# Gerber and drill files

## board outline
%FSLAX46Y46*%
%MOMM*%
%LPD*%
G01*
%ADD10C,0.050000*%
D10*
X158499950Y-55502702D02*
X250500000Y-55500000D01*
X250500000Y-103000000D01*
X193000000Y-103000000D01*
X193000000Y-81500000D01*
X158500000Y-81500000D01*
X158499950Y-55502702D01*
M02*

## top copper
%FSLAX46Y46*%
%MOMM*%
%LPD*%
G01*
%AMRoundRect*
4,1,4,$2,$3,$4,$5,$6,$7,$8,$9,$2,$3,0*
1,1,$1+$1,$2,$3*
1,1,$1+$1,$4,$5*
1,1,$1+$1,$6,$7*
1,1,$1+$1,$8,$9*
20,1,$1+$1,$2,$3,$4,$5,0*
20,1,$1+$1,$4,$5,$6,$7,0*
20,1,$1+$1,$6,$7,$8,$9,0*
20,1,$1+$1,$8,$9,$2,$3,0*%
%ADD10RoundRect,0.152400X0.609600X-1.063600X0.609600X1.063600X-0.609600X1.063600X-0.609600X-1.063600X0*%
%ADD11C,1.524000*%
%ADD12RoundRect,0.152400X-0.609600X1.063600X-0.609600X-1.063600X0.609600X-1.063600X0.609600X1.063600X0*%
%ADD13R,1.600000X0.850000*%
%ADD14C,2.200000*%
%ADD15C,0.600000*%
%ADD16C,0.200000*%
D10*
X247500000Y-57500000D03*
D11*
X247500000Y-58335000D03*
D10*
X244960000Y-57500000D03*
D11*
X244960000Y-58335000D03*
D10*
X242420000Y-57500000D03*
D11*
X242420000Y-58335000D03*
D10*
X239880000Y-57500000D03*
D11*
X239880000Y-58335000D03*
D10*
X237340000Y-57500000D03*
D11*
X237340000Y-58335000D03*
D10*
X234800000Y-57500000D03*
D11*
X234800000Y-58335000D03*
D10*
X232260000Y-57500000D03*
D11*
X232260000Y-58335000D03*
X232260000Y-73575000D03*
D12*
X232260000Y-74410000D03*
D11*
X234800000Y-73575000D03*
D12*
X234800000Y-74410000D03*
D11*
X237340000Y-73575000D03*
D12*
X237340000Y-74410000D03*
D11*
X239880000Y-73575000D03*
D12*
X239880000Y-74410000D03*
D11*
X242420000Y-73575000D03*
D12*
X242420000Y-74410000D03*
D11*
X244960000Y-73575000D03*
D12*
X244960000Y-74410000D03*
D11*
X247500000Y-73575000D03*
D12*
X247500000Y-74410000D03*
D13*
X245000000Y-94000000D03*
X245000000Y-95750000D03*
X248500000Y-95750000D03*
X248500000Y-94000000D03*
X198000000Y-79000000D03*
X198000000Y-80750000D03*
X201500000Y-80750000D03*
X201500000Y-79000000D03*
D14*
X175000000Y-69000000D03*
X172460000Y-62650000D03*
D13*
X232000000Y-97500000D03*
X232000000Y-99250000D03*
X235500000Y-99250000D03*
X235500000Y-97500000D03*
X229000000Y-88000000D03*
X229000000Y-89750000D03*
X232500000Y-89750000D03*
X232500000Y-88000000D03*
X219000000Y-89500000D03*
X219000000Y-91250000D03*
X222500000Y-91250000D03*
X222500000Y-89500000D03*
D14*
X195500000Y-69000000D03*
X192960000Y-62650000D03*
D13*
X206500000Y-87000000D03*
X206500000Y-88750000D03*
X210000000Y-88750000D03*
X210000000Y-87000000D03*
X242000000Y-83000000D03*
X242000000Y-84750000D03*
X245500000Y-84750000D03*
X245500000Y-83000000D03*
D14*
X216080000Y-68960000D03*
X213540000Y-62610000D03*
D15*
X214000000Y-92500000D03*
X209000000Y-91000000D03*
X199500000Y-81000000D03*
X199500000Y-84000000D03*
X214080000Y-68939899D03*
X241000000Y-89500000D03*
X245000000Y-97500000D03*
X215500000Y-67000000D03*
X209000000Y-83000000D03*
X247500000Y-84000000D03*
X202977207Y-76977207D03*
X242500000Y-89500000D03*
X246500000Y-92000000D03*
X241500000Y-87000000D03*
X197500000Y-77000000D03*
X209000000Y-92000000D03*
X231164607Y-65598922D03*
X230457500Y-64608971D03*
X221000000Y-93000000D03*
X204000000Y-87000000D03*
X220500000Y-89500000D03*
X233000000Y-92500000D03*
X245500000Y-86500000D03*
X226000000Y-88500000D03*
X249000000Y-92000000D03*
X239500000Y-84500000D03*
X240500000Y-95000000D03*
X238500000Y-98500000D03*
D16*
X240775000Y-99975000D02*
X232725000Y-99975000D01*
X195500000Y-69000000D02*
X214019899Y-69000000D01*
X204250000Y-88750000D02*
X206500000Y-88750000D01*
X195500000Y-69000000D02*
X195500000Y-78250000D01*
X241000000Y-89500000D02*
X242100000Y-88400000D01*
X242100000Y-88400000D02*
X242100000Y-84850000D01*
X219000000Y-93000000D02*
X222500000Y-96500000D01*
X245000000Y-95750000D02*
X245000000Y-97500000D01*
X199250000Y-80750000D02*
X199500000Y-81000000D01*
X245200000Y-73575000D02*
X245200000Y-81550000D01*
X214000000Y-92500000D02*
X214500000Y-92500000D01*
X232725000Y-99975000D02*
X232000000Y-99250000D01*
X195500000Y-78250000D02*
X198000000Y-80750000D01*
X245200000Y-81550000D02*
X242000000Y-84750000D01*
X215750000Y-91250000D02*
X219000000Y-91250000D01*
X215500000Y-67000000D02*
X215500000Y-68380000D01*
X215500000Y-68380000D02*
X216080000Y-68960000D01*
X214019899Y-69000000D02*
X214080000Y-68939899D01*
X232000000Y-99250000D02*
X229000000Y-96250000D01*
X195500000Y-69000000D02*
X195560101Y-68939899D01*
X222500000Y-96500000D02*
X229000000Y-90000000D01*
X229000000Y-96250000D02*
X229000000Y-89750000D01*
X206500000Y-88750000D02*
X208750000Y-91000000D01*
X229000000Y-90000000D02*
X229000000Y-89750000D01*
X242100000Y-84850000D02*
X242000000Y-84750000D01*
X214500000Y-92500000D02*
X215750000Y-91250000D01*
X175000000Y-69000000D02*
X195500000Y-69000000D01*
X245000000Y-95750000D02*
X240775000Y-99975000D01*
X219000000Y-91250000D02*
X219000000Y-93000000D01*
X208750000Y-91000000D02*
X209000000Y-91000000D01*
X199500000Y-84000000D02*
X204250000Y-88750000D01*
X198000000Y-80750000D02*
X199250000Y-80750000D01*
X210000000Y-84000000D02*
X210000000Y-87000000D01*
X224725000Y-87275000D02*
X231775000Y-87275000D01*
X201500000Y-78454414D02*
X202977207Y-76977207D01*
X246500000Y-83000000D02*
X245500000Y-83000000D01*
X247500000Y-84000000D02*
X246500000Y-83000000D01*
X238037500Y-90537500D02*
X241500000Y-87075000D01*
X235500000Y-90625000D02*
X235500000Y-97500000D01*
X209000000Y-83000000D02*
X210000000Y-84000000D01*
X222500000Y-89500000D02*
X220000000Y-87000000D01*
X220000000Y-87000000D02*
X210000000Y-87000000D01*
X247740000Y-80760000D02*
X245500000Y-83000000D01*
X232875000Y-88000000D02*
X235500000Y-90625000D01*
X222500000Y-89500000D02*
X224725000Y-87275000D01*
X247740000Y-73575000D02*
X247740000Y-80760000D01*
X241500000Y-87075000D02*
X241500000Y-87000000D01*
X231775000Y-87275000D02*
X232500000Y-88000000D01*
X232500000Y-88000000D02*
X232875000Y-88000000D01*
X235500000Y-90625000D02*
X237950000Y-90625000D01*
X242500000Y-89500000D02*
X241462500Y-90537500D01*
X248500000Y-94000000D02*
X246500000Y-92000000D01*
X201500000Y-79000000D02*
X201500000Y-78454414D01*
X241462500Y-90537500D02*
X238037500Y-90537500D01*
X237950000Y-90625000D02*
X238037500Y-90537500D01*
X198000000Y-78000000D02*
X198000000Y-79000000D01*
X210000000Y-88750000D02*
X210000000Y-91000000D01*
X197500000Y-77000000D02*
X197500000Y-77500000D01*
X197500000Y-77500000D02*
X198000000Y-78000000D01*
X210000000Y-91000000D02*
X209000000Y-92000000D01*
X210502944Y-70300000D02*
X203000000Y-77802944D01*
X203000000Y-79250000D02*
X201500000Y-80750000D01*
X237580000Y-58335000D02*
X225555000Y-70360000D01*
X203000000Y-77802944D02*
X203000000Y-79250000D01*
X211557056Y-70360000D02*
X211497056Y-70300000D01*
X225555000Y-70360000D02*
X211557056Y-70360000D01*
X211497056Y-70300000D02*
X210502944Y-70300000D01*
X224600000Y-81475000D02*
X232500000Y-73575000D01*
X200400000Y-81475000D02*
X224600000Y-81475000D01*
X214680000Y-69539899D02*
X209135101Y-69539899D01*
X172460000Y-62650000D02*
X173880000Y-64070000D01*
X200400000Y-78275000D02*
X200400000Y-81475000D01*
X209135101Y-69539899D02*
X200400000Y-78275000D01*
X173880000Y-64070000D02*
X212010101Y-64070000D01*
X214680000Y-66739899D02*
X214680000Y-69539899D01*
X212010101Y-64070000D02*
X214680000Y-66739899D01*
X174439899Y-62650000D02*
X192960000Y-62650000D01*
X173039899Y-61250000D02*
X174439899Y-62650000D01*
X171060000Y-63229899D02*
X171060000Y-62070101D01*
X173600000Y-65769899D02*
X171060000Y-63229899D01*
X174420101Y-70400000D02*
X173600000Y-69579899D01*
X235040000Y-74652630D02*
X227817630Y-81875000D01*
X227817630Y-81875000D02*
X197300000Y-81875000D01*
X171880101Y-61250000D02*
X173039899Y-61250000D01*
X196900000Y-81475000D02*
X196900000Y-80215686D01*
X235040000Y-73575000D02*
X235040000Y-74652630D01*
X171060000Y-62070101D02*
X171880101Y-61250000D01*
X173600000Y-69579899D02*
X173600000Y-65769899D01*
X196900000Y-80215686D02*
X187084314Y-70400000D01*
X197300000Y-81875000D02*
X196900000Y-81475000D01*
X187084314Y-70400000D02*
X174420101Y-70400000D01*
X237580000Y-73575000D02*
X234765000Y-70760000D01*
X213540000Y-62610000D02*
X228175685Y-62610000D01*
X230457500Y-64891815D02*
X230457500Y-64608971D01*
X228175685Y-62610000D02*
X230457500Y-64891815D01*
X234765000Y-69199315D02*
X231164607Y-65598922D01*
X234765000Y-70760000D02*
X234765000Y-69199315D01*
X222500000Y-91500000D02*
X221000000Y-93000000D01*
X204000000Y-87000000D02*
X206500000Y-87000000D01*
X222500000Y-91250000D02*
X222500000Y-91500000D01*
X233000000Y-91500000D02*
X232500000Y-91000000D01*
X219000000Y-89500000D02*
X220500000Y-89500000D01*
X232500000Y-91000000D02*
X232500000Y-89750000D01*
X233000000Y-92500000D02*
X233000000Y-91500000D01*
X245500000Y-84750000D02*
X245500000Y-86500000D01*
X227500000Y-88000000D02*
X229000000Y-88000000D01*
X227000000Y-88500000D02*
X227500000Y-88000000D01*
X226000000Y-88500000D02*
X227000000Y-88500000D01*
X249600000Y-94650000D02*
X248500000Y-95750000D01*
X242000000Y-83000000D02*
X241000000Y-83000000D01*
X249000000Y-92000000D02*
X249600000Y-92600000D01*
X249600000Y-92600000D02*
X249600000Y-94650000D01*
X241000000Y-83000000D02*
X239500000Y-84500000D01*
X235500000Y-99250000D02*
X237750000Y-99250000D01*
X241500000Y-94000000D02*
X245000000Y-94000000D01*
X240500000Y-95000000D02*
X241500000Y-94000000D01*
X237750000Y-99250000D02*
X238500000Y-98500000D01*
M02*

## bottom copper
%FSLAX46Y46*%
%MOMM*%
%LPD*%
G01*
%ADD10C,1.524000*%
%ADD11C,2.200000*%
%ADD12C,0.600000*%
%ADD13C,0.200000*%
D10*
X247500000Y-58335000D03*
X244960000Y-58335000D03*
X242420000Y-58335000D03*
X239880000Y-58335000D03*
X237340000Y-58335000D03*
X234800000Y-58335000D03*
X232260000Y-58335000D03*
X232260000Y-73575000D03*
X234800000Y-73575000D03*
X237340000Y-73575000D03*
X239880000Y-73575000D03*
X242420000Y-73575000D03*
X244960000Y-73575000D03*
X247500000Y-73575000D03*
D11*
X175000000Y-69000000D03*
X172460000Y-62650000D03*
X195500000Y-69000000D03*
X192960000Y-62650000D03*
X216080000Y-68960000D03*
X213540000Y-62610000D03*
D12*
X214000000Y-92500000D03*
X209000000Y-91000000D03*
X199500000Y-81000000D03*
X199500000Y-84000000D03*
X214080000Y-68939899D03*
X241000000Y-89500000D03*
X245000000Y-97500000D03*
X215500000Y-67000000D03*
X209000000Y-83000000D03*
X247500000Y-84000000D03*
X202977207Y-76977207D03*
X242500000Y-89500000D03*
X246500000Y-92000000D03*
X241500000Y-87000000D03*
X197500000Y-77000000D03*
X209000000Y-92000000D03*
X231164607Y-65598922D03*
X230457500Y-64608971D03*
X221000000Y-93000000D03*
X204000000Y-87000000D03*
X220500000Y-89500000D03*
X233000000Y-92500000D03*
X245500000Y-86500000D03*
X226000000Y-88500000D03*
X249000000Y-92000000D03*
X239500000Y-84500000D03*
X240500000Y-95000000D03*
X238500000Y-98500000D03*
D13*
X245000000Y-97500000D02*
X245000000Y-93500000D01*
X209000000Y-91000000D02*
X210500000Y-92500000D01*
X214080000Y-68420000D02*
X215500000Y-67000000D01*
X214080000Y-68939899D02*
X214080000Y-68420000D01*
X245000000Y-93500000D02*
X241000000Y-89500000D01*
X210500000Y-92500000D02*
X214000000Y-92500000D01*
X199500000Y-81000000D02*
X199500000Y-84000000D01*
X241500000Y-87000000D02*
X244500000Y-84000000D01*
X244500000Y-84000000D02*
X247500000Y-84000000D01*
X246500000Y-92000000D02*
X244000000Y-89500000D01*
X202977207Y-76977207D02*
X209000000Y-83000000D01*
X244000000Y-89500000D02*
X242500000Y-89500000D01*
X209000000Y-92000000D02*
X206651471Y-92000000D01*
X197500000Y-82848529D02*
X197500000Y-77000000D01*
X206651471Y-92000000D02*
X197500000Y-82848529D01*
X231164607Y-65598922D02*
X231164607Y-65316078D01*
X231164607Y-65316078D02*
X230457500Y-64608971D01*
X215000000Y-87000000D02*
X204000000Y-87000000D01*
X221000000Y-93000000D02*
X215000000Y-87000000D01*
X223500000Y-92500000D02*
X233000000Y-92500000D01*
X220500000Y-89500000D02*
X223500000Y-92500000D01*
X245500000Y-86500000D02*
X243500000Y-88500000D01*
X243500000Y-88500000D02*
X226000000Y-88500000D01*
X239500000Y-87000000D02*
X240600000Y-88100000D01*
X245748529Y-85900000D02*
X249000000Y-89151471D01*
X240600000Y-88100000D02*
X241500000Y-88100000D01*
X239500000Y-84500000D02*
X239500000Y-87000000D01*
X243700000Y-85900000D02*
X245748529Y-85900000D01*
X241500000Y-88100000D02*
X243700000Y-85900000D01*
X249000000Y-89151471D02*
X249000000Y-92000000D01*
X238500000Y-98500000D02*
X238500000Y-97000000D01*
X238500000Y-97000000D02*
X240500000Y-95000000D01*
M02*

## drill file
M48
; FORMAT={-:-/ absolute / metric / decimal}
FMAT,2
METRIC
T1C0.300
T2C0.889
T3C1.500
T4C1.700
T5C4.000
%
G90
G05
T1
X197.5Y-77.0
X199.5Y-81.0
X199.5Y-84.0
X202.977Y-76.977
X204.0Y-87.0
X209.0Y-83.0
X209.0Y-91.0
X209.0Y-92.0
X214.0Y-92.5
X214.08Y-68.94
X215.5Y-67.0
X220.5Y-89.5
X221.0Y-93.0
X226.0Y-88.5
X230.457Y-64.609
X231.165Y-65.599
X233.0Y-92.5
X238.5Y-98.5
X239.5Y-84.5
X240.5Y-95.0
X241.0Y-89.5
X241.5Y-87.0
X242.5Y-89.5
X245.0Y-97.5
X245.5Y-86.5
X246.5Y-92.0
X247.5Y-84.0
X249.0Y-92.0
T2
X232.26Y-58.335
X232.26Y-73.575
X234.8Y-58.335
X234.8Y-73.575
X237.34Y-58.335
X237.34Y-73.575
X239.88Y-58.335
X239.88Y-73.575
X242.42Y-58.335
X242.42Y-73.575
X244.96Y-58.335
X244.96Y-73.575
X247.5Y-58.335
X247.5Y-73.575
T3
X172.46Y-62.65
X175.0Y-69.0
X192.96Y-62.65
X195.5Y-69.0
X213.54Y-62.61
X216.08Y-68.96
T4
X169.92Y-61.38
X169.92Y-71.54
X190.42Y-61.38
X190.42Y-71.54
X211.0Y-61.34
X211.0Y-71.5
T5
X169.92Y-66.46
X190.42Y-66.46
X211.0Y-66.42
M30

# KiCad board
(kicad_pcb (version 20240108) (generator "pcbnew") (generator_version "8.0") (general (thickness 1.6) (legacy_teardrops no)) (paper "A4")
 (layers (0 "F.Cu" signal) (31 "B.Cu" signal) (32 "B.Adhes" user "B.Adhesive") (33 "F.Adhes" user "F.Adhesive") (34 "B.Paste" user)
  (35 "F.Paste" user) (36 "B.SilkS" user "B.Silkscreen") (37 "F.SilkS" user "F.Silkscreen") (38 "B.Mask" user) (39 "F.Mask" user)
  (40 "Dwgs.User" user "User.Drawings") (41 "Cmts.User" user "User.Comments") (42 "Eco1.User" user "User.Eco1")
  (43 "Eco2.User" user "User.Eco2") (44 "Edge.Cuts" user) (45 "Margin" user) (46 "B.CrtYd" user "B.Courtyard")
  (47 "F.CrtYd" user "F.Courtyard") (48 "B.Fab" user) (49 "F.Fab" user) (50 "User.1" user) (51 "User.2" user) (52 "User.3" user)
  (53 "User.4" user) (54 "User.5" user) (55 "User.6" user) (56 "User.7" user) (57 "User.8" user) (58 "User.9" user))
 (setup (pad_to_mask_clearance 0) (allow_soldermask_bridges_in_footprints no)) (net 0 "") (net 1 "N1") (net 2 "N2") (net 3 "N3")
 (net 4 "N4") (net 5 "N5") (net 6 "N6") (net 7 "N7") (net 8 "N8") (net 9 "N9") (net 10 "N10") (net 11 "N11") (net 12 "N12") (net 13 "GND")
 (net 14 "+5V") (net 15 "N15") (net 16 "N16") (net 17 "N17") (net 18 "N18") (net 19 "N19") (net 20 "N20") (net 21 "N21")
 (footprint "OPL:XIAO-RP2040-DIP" (layer "F.Cu") (at 239.88 65.955 -90)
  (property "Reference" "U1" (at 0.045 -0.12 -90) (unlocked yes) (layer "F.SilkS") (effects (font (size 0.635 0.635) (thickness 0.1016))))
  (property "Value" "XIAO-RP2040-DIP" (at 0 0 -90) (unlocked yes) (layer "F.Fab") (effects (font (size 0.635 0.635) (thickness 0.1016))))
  (pad "1" smd roundrect (at -8.455 -7.62 90) (size 2.432 1.524) (layers "F.Cu" "F.Mask") (roundrect_rratio 0.1) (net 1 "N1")
   (thermal_bridge_angle 45))
  (pad "1" thru_hole circle (at -7.62 -7.62 90) (size 1.524 1.524) (drill 0.889) (layers "*.Cu" "*.Mask") (remove_unused_layers no)
   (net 1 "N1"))
  (pad "2" smd roundrect (at -8.455 -5.08 90) (size 2.432 1.524) (layers "F.Cu" "F.Mask") (roundrect_rratio 0.1) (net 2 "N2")
   (thermal_bridge_angle 45))
  (pad "2" thru_hole circle (at -7.62 -5.08 90) (size 1.524 1.524) (drill 0.889) (layers "*.Cu" "*.Mask") (remove_unused_layers no)
   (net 2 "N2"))
  (pad "3" smd roundrect (at -8.455 -2.54 90) (size 2.432 1.524) (layers "F.Cu" "F.Mask") (roundrect_rratio 0.1) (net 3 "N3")
   (thermal_bridge_angle 45))
  (pad "3" thru_hole circle (at -7.62 -2.54 90) (size 1.524 1.524) (drill 0.889) (layers "*.Cu" "*.Mask") (remove_unused_layers no)
   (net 3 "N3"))
  (pad "4" smd roundrect (at -8.455 0 90) (size 2.432 1.524) (layers "F.Cu" "F.Mask") (roundrect_rratio 0.1) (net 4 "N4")
   (thermal_bridge_angle 45))
  (pad "4" thru_hole circle (at -7.62 0 90) (size 1.524 1.524) (drill 0.889) (layers "*.Cu" "*.Mask") (remove_unused_layers no) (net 4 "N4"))
  (pad "5" smd roundrect (at -8.455 2.54 90) (size 2.432 1.524) (layers "F.Cu" "F.Mask") (roundrect_rratio 0.1) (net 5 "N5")
   (thermal_bridge_angle 45))
  (pad "5" thru_hole circle (at -7.62 2.54 90) (size 1.524 1.524) (drill 0.889) (layers "*.Cu" "*.Mask") (remove_unused_layers no)
   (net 5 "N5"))
  (pad "6" smd roundrect (at -8.455 5.08 90) (size 2.432 1.524) (layers "F.Cu" "F.Mask") (roundrect_rratio 0.1) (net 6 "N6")
   (thermal_bridge_angle 45))
  (pad "6" thru_hole circle (at -7.62 5.08 90) (size 1.524 1.524) (drill 0.889) (layers "*.Cu" "*.Mask") (remove_unused_layers no)
   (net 6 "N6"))
  (pad "7" smd roundrect (at -8.455 7.62 90) (size 2.432 1.524) (layers "F.Cu" "F.Mask") (roundrect_rratio 0.1) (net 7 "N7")
   (thermal_bridge_angle 45))
  (pad "7" thru_hole circle (at -7.62 7.62 90) (size 1.524 1.524) (drill 0.889) (layers "*.Cu" "*.Mask") (remove_unused_layers no)
   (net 7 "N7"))
  (pad "8" thru_hole circle (at 7.62 7.62 270) (size 1.524 1.524) (drill 0.889) (layers "*.Cu" "*.Mask") (remove_unused_layers no)
   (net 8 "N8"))
  (pad "8" smd roundrect (at 8.455 7.62 270) (size 2.432 1.524) (layers "F.Cu" "F.Mask") (roundrect_rratio 0.1) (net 8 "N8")
   (thermal_bridge_angle 45))
  (pad "9" thru_hole circle (at 7.62 5.08 270) (size 1.524 1.524) (drill 0.889) (layers "*.Cu" "*.Mask") (remove_unused_layers no)
   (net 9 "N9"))
  (pad "9" smd roundrect (at 8.455 5.08 270) (size 2.432 1.524) (layers "F.Cu" "F.Mask") (roundrect_rratio 0.1) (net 9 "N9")
   (thermal_bridge_angle 45))
  (pad "10" thru_hole circle (at 7.62 2.54 270) (size 1.524 1.524) (drill 0.889) (layers "*.Cu" "*.Mask") (remove_unused_layers no)
   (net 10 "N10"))
  (pad "10" smd roundrect (at 8.455 2.54 270) (size 2.432 1.524) (layers "F.Cu" "F.Mask") (roundrect_rratio 0.1) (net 10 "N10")
   (thermal_bridge_angle 45))
  (pad "11" thru_hole circle (at 7.62 0 270) (size 1.524 1.524) (drill 0.889) (layers "*.Cu" "*.Mask") (remove_unused_layers no)
   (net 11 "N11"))
  (pad "11" smd roundrect (at 8.455 0 270) (size 2.432 1.524) (layers "F.Cu" "F.Mask") (roundrect_rratio 0.1) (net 11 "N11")
   (thermal_bridge_angle 45))
  (pad "12" thru_hole circle (at 7.62 -2.54 270) (size 1.524 1.524) (drill 0.889) (layers "*.Cu" "*.Mask") (remove_unused_layers no)
   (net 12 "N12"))
  (pad "12" smd roundrect (at 8.455 -2.54 270) (size 2.432 1.524) (layers "F.Cu" "F.Mask") (roundrect_rratio 0.1) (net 12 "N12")
   (thermal_bridge_angle 45))
  (pad "13" thru_hole circle (at 7.62 -5.08 270) (size 1.524 1.524) (drill 0.889) (layers "*.Cu" "*.Mask") (remove_unused_layers no)
   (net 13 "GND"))
  (pad "13" smd roundrect (at 8.455 -5.08 270) (size 2.432 1.524) (layers "F.Cu" "F.Mask") (roundrect_rratio 0.1) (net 13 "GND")
   (thermal_bridge_angle 45))
  (pad "14" thru_hole circle (at 7.62 -7.62 270) (size 1.524 1.524) (drill 0.889) (layers "*.Cu" "*.Mask") (remove_unused_layers no)
   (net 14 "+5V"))
  (pad "14" smd roundrect (at 8.455 -7.62 270) (size 2.432 1.524) (layers "F.Cu" "F.Mask") (roundrect_rratio 0.1) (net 14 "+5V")
   (thermal_bridge_angle 45)))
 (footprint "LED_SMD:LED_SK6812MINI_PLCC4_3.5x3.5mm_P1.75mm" (layer "F.Cu") (at 246.75 94.875)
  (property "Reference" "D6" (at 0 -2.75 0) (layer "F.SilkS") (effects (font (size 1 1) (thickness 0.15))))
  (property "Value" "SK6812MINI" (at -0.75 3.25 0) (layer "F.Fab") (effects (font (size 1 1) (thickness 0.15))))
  (pad "1" smd rect (at -1.75 -0.875) (size 1.6 0.85) (layers "F.Cu" "F.Paste" "F.Mask") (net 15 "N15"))
  (pad "2" smd rect (at -1.75 0.875) (size 1.6 0.85) (layers "F.Cu" "F.Paste" "F.Mask") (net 13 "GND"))
  (pad "3" smd rect (at 1.75 0.875) (size 1.6 0.85) (layers "F.Cu" "F.Paste" "F.Mask") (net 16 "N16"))
  (pad "4" smd rect (at 1.75 -0.875) (size 1.6 0.85) (layers "F.Cu" "F.Paste" "F.Mask") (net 14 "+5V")))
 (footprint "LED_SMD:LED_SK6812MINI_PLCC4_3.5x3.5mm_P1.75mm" (layer "F.Cu") (at 199.75 79.875)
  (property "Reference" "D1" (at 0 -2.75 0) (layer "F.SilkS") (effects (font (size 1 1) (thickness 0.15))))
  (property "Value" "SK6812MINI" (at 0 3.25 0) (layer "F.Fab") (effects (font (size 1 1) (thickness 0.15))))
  (pad "1" smd rect (at -1.75 -0.875) (size 1.6 0.85) (layers "F.Cu" "F.Paste" "F.Mask") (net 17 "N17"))
  (pad "2" smd rect (at -1.75 0.875) (size 1.6 0.85) (layers "F.Cu" "F.Paste" "F.Mask") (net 13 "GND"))
  (pad "3" smd rect (at 1.75 0.875) (size 1.6 0.85) (layers "F.Cu" "F.Paste" "F.Mask") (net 5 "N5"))
  (pad "4" smd rect (at 1.75 -0.875) (size 1.6 0.85) (layers "F.Cu" "F.Paste" "F.Mask") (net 14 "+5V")))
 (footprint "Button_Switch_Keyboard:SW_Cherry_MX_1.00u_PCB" (layer "F.Cu") (at 175 69 -90)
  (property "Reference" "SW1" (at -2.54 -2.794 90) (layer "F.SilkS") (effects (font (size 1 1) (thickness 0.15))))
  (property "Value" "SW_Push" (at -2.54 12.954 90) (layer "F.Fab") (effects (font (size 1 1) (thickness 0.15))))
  (pad "" np_thru_hole circle (at -7.62 5.08 270) (size 1.7 1.7) (drill 1.7) (layers "*.Cu" "*.Mask"))
  (pad "" np_thru_hole circle (at -2.54 5.08 270) (size 4 4) (drill 4) (layers "*.Cu" "*.Mask"))
  (pad "" np_thru_hole circle (at 2.54 5.08 270) (size 1.7 1.7) (drill 1.7) (layers "*.Cu" "*.Mask"))
  (pad "1" thru_hole circle (at 0 0 270) (size 2.2 2.2) (drill 1.5) (layers "*.Cu" "*.Mask") (remove_unused_layers no) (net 13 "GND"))
  (pad "2" thru_hole circle (at -6.35 2.54 270) (size 2.2 2.2) (drill 1.5) (layers "*.Cu" "*.Mask") (remove_unused_layers no) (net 8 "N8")))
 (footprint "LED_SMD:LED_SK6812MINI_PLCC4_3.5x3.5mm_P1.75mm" (layer "F.Cu") (at 233.75 98.375)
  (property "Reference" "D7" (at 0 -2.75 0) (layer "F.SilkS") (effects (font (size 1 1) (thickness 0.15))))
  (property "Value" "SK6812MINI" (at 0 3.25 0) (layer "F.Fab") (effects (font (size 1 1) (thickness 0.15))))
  (pad "1" smd rect (at -1.75 -0.875) (size 1.6 0.85) (layers "F.Cu" "F.Paste" "F.Mask") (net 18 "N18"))
  (pad "2" smd rect (at -1.75 0.875) (size 1.6 0.85) (layers "F.Cu" "F.Paste" "F.Mask") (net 13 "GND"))
  (pad "3" smd rect (at 1.75 0.875) (size 1.6 0.85) (layers "F.Cu" "F.Paste" "F.Mask") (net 15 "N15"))
  (pad "4" smd rect (at 1.75 -0.875) (size 1.6 0.85) (layers "F.Cu" "F.Paste" "F.Mask") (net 14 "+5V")))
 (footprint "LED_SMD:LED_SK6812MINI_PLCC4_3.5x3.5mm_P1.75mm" (layer "F.Cu") (at 230.75 88.875)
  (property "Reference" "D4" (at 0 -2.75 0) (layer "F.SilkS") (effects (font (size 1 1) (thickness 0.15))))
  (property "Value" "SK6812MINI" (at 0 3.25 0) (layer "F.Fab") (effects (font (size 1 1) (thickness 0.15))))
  (pad "1" smd rect (at -1.75 -0.875) (size 1.6 0.85) (layers "F.Cu" "F.Paste" "F.Mask") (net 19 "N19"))
  (pad "2" smd rect (at -1.75 0.875) (size 1.6 0.85) (layers "F.Cu" "F.Paste" "F.Mask") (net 13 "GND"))
  (pad "3" smd rect (at 1.75 0.875) (size 1.6 0.85) (layers "F.Cu" "F.Paste" "F.Mask") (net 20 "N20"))
  (pad "4" smd rect (at 1.75 -0.875) (size 1.6 0.85) (layers "F.Cu" "F.Paste" "F.Mask") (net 14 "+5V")))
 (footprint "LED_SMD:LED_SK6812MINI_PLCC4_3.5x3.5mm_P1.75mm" (layer "F.Cu") (at 220.75 90.375)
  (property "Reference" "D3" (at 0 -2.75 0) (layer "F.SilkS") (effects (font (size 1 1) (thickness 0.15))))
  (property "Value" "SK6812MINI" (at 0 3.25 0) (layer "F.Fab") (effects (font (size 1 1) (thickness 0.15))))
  (pad "1" smd rect (at -1.75 -0.875) (size 1.6 0.85) (layers "F.Cu" "F.Paste" "F.Mask") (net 20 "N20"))
  (pad "2" smd rect (at -1.75 0.875) (size 1.6 0.85) (layers "F.Cu" "F.Paste" "F.Mask") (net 13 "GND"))
  (pad "3" smd rect (at 1.75 0.875) (size 1.6 0.85) (layers "F.Cu" "F.Paste" "F.Mask") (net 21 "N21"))
  (pad "4" smd rect (at 1.75 -0.875) (size 1.6 0.85) (layers "F.Cu" "F.Paste" "F.Mask") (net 14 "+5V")))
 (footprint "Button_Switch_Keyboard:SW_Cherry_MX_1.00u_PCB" (layer "F.Cu") (at 195.5 69 -90)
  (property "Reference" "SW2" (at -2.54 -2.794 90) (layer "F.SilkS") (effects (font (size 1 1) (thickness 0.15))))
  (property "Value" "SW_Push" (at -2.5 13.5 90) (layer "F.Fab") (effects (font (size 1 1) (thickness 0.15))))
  (pad "" np_thru_hole circle (at -7.62 5.08 270) (size 1.7 1.7) (drill 1.7) (layers "*.Cu" "*.Mask"))
  (pad "" np_thru_hole circle (at -2.54 5.08 270) (size 4 4) (drill 4) (layers "*.Cu" "*.Mask"))
  (pad "" np_thru_hole circle (at 2.54 5.08 270) (size 1.7 1.7) (drill 1.7) (layers "*.Cu" "*.Mask"))
  (pad "1" thru_hole circle (at 0 0 270) (size 2.2 2.2) (drill 1.5) (layers "*.Cu" "*.Mask") (remove_unused_layers no) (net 13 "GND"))
  (pad "2" thru_hole circle (at -6.35 2.54 270) (size 2.2 2.2) (drill 1.5) (layers "*.Cu" "*.Mask") (remove_unused_layers no) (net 9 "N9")))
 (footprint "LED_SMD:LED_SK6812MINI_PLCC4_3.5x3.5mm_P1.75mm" (layer "F.Cu") (at 208.25 87.875)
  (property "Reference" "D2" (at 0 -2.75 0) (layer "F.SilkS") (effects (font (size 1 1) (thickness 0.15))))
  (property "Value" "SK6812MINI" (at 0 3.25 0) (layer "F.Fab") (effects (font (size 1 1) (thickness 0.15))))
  (pad "1" smd rect (at -1.75 -0.875) (size 1.6 0.85) (layers "F.Cu" "F.Paste" "F.Mask") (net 21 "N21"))
  (pad "2" smd rect (at -1.75 0.875) (size 1.6 0.85) (layers "F.Cu" "F.Paste" "F.Mask") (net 13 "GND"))
  (pad "3" smd rect (at 1.75 0.875) (size 1.6 0.85) (layers "F.Cu" "F.Paste" "F.Mask") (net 17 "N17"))
  (pad "4" smd rect (at 1.75 -0.875) (size 1.6 0.85) (layers "F.Cu" "F.Paste" "F.Mask") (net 14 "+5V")))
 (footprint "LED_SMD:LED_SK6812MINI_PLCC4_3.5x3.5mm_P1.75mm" (layer "F.Cu") (at 243.75 83.875)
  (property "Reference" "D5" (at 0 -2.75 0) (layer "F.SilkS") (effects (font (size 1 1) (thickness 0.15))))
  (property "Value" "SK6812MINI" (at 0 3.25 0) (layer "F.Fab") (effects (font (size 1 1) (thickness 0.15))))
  (pad "1" smd rect (at -1.75 -0.875) (size 1.6 0.85) (layers "F.Cu" "F.Paste" "F.Mask") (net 16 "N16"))
  (pad "2" smd rect (at -1.75 0.875) (size 1.6 0.85) (layers "F.Cu" "F.Paste" "F.Mask") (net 13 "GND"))
  (pad "3" smd rect (at 1.75 0.875) (size 1.6 0.85) (layers "F.Cu" "F.Paste" "F.Mask") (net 19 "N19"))
  (pad "4" smd rect (at 1.75 -0.875) (size 1.6 0.85) (layers "F.Cu" "F.Paste" "F.Mask") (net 14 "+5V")))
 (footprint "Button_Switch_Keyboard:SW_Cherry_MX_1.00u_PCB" (layer "F.Cu") (at 216.08 68.96 -90)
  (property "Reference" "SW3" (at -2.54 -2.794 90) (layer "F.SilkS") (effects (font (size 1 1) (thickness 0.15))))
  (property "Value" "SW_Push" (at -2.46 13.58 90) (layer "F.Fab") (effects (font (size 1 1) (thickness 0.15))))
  (pad "" np_thru_hole circle (at -7.62 5.08 270) (size 1.7 1.7) (drill 1.7) (layers "*.Cu" "*.Mask"))
  (pad "" np_thru_hole circle (at -2.54 5.08 270) (size 4 4) (drill 4) (layers "*.Cu" "*.Mask"))
  (pad "" np_thru_hole circle (at 2.54 5.08 270) (size 1.7 1.7) (drill 1.7) (layers "*.Cu" "*.Mask"))
  (pad "1" thru_hole circle (at 0 0 270) (size 2.2 2.2) (drill 1.5) (layers "*.Cu" "*.Mask") (remove_unused_layers no) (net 13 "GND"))
  (pad "2" thru_hole circle (at -6.35 2.54 270) (size 2.2 2.2) (drill 1.5) (layers "*.Cu" "*.Mask") (remove_unused_layers no) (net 10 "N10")))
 (gr_poly
  (pts (xy 158.49995 55.502702) (xy 250.5 55.5) (xy 250.5 103) (xy 193 103) (xy 193 81.5) (xy 158.5 81.5))
  (stroke (width 0.05) (type solid)) (fill none) (layer "Edge.Cuts"))
 (segment (start 240.775 99.975) (end 232.725 99.975) (width 0.2) (layer "F.Cu") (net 13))
 (segment (start 195.5 69) (end 214.019899 69) (width 0.2) (layer "F.Cu") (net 13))
 (segment (start 204.25 88.75) (end 206.5 88.75) (width 0.2) (layer "F.Cu") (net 13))
 (segment (start 195.5 69) (end 195.5 78.25) (width 0.2) (layer "F.Cu") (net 13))
 (segment (start 241 89.5) (end 242.1 88.4) (width 0.2) (layer "F.Cu") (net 13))
 (segment (start 242.1 88.4) (end 242.1 84.85) (width 0.2) (layer "F.Cu") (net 13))
 (segment (start 219 93) (end 222.5 96.5) (width 0.2) (layer "F.Cu") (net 13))
 (segment (start 245 95.75) (end 245 97.5) (width 0.2) (layer "F.Cu") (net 13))
 (segment (start 199.25 80.75) (end 199.5 81) (width 0.2) (layer "F.Cu") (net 13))
 (segment (start 245.2 73.575) (end 245.2 81.55) (width 0.2) (layer "F.Cu") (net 13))
 (segment (start 214 92.5) (end 214.5 92.5) (width 0.2) (layer "F.Cu") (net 13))
 (segment (start 232.725 99.975) (end 232 99.25) (width 0.2) (layer "F.Cu") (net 13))
 (segment (start 195.5 78.25) (end 198 80.75) (width 0.2) (layer "F.Cu") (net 13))
 (segment (start 245.2 81.55) (end 242 84.75) (width 0.2) (layer "F.Cu") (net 13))
 (segment (start 215.75 91.25) (end 219 91.25) (width 0.2) (layer "F.Cu") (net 13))
 (segment (start 215.5 67) (end 215.5 68.38) (width 0.2) (layer "F.Cu") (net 13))
 (segment (start 215.5 68.38) (end 216.08 68.96) (width 0.2) (layer "F.Cu") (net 13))
 (segment (start 214.019899 69) (end 214.08 68.939899) (width 0.2) (layer "F.Cu") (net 13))
 (segment (start 232 99.25) (end 229 96.25) (width 0.2) (layer "F.Cu") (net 13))
 (segment (start 195.5 69) (end 195.560101 68.939899) (width 0.2) (layer "F.Cu") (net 13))
 (segment (start 222.5 96.5) (end 229 90) (width 0.2) (layer "F.Cu") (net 13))
 (segment (start 229 96.25) (end 229 89.75) (width 0.2) (layer "F.Cu") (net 13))
 (segment (start 206.5 88.75) (end 208.75 91) (width 0.2) (layer "F.Cu") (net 13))
 (segment (start 229 90) (end 229 89.75) (width 0.2) (layer "F.Cu") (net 13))
 (segment (start 242.1 84.85) (end 242 84.75) (width 0.2) (layer "F.Cu") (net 13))
 (segment (start 214.5 92.5) (end 215.75 91.25) (width 0.2) (layer "F.Cu") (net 13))
 (segment (start 175 69) (end 195.5 69) (width 0.2) (layer "F.Cu") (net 13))
 (segment (start 245 95.75) (end 240.775 99.975) (width 0.2) (layer "F.Cu") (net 13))
 (segment (start 219 91.25) (end 219 93) (width 0.2) (layer "F.Cu") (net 13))
 (segment (start 208.75 91) (end 209 91) (width 0.2) (layer "F.Cu") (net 13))
 (segment (start 199.5 84) (end 204.25 88.75) (width 0.2) (layer "F.Cu") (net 13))
 (segment (start 198 80.75) (end 199.25 80.75) (width 0.2) (layer "F.Cu") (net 13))
 (via (at 214 92.5) (size 0.6) (drill 0.3) (layers "F.Cu" "B.Cu") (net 13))
 (via (at 209 91) (size 0.6) (drill 0.3) (layers "F.Cu" "B.Cu") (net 13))
 (via (at 199.5 81) (size 0.6) (drill 0.3) (layers "F.Cu" "B.Cu") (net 13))
 (via (at 199.5 84) (size 0.6) (drill 0.3) (layers "F.Cu" "B.Cu") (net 13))
 (via (at 214.08 68.939899) (size 0.6) (drill 0.3) (layers "F.Cu" "B.Cu") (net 13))
 (via (at 241 89.5) (size 0.6) (drill 0.3) (layers "F.Cu" "B.Cu") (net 13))
 (via (at 245 97.5) (size 0.6) (drill 0.3) (layers "F.Cu" "B.Cu") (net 13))
 (via (at 215.5 67) (size 0.6) (drill 0.3) (layers "F.Cu" "B.Cu") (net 13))
 (segment (start 245 97.5) (end 245 93.5) (width 0.2) (layer "B.Cu") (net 13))
 (segment (start 209 91) (end 210.5 92.5) (width 0.2) (layer "B.Cu") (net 13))
 (segment (start 214.08 68.42) (end 215.5 67) (width 0.2) (layer "B.Cu") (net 13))
 (segment (start 214.08 68.939899) (end 214.08 68.42) (width 0.2) (layer "B.Cu") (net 13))
 (segment (start 245 93.5) (end 241 89.5) (width 0.2) (layer "B.Cu") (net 13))
 (segment (start 210.5 92.5) (end 214 92.5) (width 0.2) (layer "B.Cu") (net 13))
 (segment (start 199.5 81) (end 199.5 84) (width 0.2) (layer "B.Cu") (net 13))
 (segment (start 210 84) (end 210 87) (width 0.2) (layer "F.Cu") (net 14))
 (segment (start 224.725 87.275) (end 231.775 87.275) (width 0.2) (layer "F.Cu") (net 14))
 (segment (start 201.5 78.454414) (end 202.977207 76.977207) (width 0.2) (layer "F.Cu") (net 14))
 (segment (start 246.5 83) (end 245.5 83) (width 0.2) (layer "F.Cu") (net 14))
 (segment (start 247.5 84) (end 246.5 83) (width 0.2) (layer "F.Cu") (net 14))
 (segment (start 238.0375 90.5375) (end 241.5 87.075) (width 0.2) (layer "F.Cu") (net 14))
 (segment (start 235.5 90.625) (end 235.5 97.5) (width 0.2) (layer "F.Cu") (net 14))
 (segment (start 209 83) (end 210 84) (width 0.2) (layer "F.Cu") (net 14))
 (segment (start 222.5 89.5) (end 220 87) (width 0.2) (layer "F.Cu") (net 14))
 (segment (start 220 87) (end 210 87) (width 0.2) (layer "F.Cu") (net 14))
 (segment (start 247.74 80.76) (end 245.5 83) (width 0.2) (layer "F.Cu") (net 14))
 (segment (start 232.875 88) (end 235.5 90.625) (width 0.2) (layer "F.Cu") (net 14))
 (segment (start 222.5 89.5) (end 224.725 87.275) (width 0.2) (layer "F.Cu") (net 14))
 (segment (start 247.74 73.575) (end 247.74 80.76) (width 0.2) (layer "F.Cu") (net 14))
 (segment (start 241.5 87.075) (end 241.5 87) (width 0.2) (layer "F.Cu") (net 14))
 (segment (start 231.775 87.275) (end 232.5 88) (width 0.2) (layer "F.Cu") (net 14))
 (segment (start 232.5 88) (end 232.875 88) (width 0.2) (layer "F.Cu") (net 14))
 (segment (start 235.5 90.625) (end 237.95 90.625) (width 0.2) (layer "F.Cu") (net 14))
 (segment (start 242.5 89.5) (end 241.4625 90.5375) (width 0.2) (layer "F.Cu") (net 14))
 (segment (start 248.5 94) (end 246.5 92) (width 0.2) (layer "F.Cu") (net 14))
 (segment (start 201.5 79) (end 201.5 78.454414) (width 0.2) (layer "F.Cu") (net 14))
 (segment (start 241.4625 90.5375) (end 238.0375 90.5375) (width 0.2) (layer "F.Cu") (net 14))
 (segment (start 237.95 90.625) (end 238.0375 90.5375) (width 0.2) (layer "F.Cu") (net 14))
 (via (at 209 83) (size 0.6) (drill 0.3) (layers "F.Cu" "B.Cu") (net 14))
 (via (at 247.5 84) (size 0.6) (drill 0.3) (layers "F.Cu" "B.Cu") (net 14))
 (via (at 202.977207 76.977207) (size 0.6) (drill 0.3) (layers "F.Cu" "B.Cu") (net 14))
 (via (at 242.5 89.5) (size 0.6) (drill 0.3) (layers "F.Cu" "B.Cu") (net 14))
 (via (at 246.5 92) (size 0.6) (drill 0.3) (layers "F.Cu" "B.Cu") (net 14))
 (via (at 241.5 87) (size 0.6) (drill 0.3) (layers "F.Cu" "B.Cu") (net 14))
 (segment (start 241.5 87) (end 244.5 84) (width 0.2) (layer "B.Cu") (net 14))
 (segment (start 244.5 84) (end 247.5 84) (width 0.2) (layer "B.Cu") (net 14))
 (segment (start 246.5 92) (end 244 89.5) (width 0.2) (layer "B.Cu") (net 14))
 (segment (start 202.977207 76.977207) (end 209 83) (width 0.2) (layer "B.Cu") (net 14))
 (segment (start 244 89.5) (end 242.5 89.5) (width 0.2) (layer "B.Cu") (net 14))
 (segment (start 198 78) (end 198 79) (width 0.2) (layer "F.Cu") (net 17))
 (segment (start 210 88.75) (end 210 91) (width 0.2) (layer "F.Cu") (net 17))
 (segment (start 197.5 77) (end 197.5 77.5) (width 0.2) (layer "F.Cu") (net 17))
 (segment (start 197.5 77.5) (end 198 78) (width 0.2) (layer "F.Cu") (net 17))
 (segment (start 210 91) (end 209 92) (width 0.2) (layer "F.Cu") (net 17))
 (via (at 197.5 77) (size 0.6) (drill 0.3) (layers "F.Cu" "B.Cu") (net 17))
 (via (at 209 92) (size 0.6) (drill 0.3) (layers "F.Cu" "B.Cu") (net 17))
 (segment (start 209 92) (end 206.651471 92) (width 0.2) (layer "B.Cu") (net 17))
 (segment (start 197.5 82.848529) (end 197.5 77) (width 0.2) (layer "B.Cu") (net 17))
 (segment (start 206.651471 92) (end 197.5 82.848529) (width 0.2) (layer "B.Cu") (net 17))
 (segment (start 210.502944 70.3) (end 203 77.802944) (width 0.2) (layer "F.Cu") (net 5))
 (segment (start 203 79.25) (end 201.5 80.75) (width 0.2) (layer "F.Cu") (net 5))
 (segment (start 237.58 58.335) (end 225.555 70.36) (width 0.2) (layer "F.Cu") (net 5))
 (segment (start 203 77.802944) (end 203 79.25) (width 0.2) (layer "F.Cu") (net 5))
 (segment (start 211.557056 70.36) (end 211.497056 70.3) (width 0.2) (layer "F.Cu") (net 5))
 (segment (start 225.555 70.36) (end 211.557056 70.36) (width 0.2) (layer "F.Cu") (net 5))
 (segment (start 211.497056 70.3) (end 210.502944 70.3) (width 0.2) (layer "F.Cu") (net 5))
 (segment (start 224.6 81.475) (end 232.5 73.575) (width 0.2) (layer "F.Cu") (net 8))
 (segment (start 200.4 81.475) (end 224.6 81.475) (width 0.2) (layer "F.Cu") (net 8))
 (segment (start 214.68 69.539899) (end 209.135101 69.539899) (width 0.2) (layer "F.Cu") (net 8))
 (segment (start 172.46 62.65) (end 173.88 64.07) (width 0.2) (layer "F.Cu") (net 8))
 (segment (start 200.4 78.275) (end 200.4 81.475) (width 0.2) (layer "F.Cu") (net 8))
 (segment (start 209.135101 69.539899) (end 200.4 78.275) (width 0.2) (layer "F.Cu") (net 8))
 (segment (start 173.88 64.07) (end 212.010101 64.07) (width 0.2) (layer "F.Cu") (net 8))
 (segment (start 214.68 66.739899) (end 214.68 69.539899) (width 0.2) (layer "F.Cu") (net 8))
 (segment (start 212.010101 64.07) (end 214.68 66.739899) (width 0.2) (layer "F.Cu") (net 8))
 (segment (start 174.439899 62.65) (end 192.96 62.65) (width 0.2) (layer "F.Cu") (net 9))
 (segment (start 173.039899 61.25) (end 174.439899 62.65) (width 0.2) (layer "F.Cu") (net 9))
 (segment (start 171.06 63.229899) (end 171.06 62.070101) (width 0.2) (layer "F.Cu") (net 9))
 (segment (start 173.6 65.769899) (end 171.06 63.229899) (width 0.2) (layer "F.Cu") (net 9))
 (segment (start 174.420101 70.4) (end 173.6 69.579899) (width 0.2) (layer "F.Cu") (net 9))
 (segment (start 235.04 74.65263) (end 227.81763 81.875) (width 0.2) (layer "F.Cu") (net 9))
 (segment (start 227.81763 81.875) (end 197.3 81.875) (width 0.2) (layer "F.Cu") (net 9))
 (segment (start 171.880101 61.25) (end 173.039899 61.25) (width 0.2) (layer "F.Cu") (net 9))
 (segment (start 196.9 81.475) (end 196.9 80.215686) (width 0.2) (layer "F.Cu") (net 9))
 (segment (start 235.04 73.575) (end 235.04 74.65263) (width 0.2) (layer "F.Cu") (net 9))
 (segment (start 171.06 62.070101) (end 171.880101 61.25) (width 0.2) (layer "F.Cu") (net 9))
 (segment (start 173.6 69.579899) (end 173.6 65.769899) (width 0.2) (layer "F.Cu") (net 9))
 (segment (start 196.9 80.215686) (end 187.084314 70.4) (width 0.2) (layer "F.Cu") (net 9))
 (segment (start 197.3 81.875) (end 196.9 81.475) (width 0.2) (layer "F.Cu") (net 9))
 (segment (start 187.084314 70.4) (end 174.420101 70.4) (width 0.2) (layer "F.Cu") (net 9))
 (segment (start 237.58 73.575) (end 234.765 70.76) (width 0.2) (layer "F.Cu") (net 10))
 (segment (start 213.54 62.61) (end 228.175685 62.61) (width 0.2) (layer "F.Cu") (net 10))
 (segment (start 230.4575 64.891815) (end 230.4575 64.608971) (width 0.2) (layer "F.Cu") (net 10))
 (segment (start 228.175685 62.61) (end 230.4575 64.891815) (width 0.2) (layer "F.Cu") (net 10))
 (segment (start 234.765 69.199315) (end 231.164607 65.598922) (width 0.2) (layer "F.Cu") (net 10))
 (segment (start 234.765 70.76) (end 234.765 69.199315) (width 0.2) (layer "F.Cu") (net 10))
 (via (at 231.164607 65.598922) (size 0.6) (drill 0.3) (layers "F.Cu" "B.Cu") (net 10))
 (via (at 230.4575 64.608971) (size 0.6) (drill 0.3) (layers "F.Cu" "B.Cu") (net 10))
 (segment (start 231.164607 65.598922) (end 231.164607 65.316078) (width 0.2) (layer "B.Cu") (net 10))
 (segment (start 231.164607 65.316078) (end 230.4575 64.608971) (width 0.2) (layer "B.Cu") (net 10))
 (segment (start 222.5 91.5) (end 221 93) (width 0.2) (layer "F.Cu") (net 21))
 (segment (start 204 87) (end 206.5 87) (width 0.2) (layer "F.Cu") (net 21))
 (segment (start 222.5 91.25) (end 222.5 91.5) (width 0.2) (layer "F.Cu") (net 21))
 (via (at 221 93) (size 0.6) (drill 0.3) (layers "F.Cu" "B.Cu") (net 21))
 (via (at 204 87) (size 0.6) (drill 0.3) (layers "F.Cu" "B.Cu") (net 21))
 (segment (start 215 87) (end 204 87) (width 0.2) (layer "B.Cu") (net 21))
 (segment (start 221 93) (end 215 87) (width 0.2) (layer "B.Cu") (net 21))
 (segment (start 233 91.5) (end 232.5 91) (width 0.2) (layer "F.Cu") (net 20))
 (segment (start 219 89.5) (end 220.5 89.5) (width 0.2) (layer "F.Cu") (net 20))
 (segment (start 232.5 91) (end 232.5 89.75) (width 0.2) (layer "F.Cu") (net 20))
 (segment (start 233 92.5) (end 233 91.5) (width 0.2) (layer "F.Cu") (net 20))
 (via (at 220.5 89.5) (size 0.6) (drill 0.3) (layers "F.Cu" "B.Cu") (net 20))
 (via (at 233 92.5) (size 0.6) (drill 0.3) (layers "F.Cu" "B.Cu") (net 20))
 (segment (start 223.5 92.5) (end 233 92.5) (width 0.2) (layer "B.Cu") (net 20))
 (segment (start 220.5 89.5) (end 223.5 92.5) (width 0.2) (layer "B.Cu") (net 20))
 (segment (start 245.5 84.75) (end 245.5 86.5) (width 0.2) (layer "F.Cu") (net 19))
 (segment (start 227.5 88) (end 229 88) (width 0.2) (layer "F.Cu") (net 19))
 (segment (start 227 88.5) (end 227.5 88) (width 0.2) (layer "F.Cu") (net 19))
 (segment (start 226 88.5) (end 227 88.5) (width 0.2) (layer "F.Cu") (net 19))
 (via (at 245.5 86.5) (size 0.6) (drill 0.3) (layers "F.Cu" "B.Cu") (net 19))
 (via (at 226 88.5) (size 0.6) (drill 0.3) (layers "F.Cu" "B.Cu") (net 19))
 (segment (start 245.5 86.5) (end 243.5 88.5) (width 0.2) (layer "B.Cu") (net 19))
 (segment (start 243.5 88.5) (end 226 88.5) (width 0.2) (layer "B.Cu") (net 19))
 (segment (start 249.6 94.65) (end 248.5 95.75) (width 0.2) (layer "F.Cu") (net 16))
 (segment (start 242 83) (end 241 83) (width 0.2) (layer "F.Cu") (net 16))
 (segment (start 249 92) (end 249.6 92.6) (width 0.2) (layer "F.Cu") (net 16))
 (segment (start 249.6 92.6) (end 249.6 94.65) (width 0.2) (layer "F.Cu") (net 16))
 (segment (start 241 83) (end 239.5 84.5) (width 0.2) (layer "F.Cu") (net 16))
 (via (at 249 92) (size 0.6) (drill 0.3) (layers "F.Cu" "B.Cu") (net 16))
 (via (at 239.5 84.5) (size 0.6) (drill 0.3) (layers "F.Cu" "B.Cu") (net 16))
 (segment (start 239.5 87) (end 240.6 88.1) (width 0.2) (layer "B.Cu") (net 16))
 (segment (start 245.748529 85.9) (end 249 89.151471) (width 0.2) (layer "B.Cu") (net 16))
 (segment (start 240.6 88.1) (end 241.5 88.1) (width 0.2) (layer "B.Cu") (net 16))
 (segment (start 239.5 84.5) (end 239.5 87) (width 0.2) (layer "B.Cu") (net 16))
 (segment (start 243.7 85.9) (end 245.748529 85.9) (width 0.2) (layer "B.Cu") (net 16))
 (segment (start 241.5 88.1) (end 243.7 85.9) (width 0.2) (layer "B.Cu") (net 16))
 (segment (start 249 89.151471) (end 249 92) (width 0.2) (layer "B.Cu") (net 16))
 (segment (start 235.5 99.25) (end 237.75 99.25) (width 0.2) (layer "F.Cu") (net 15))
 (segment (start 241.5 94) (end 245 94) (width 0.2) (layer "F.Cu") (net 15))
 (segment (start 240.5 95) (end 241.5 94) (width 0.2) (layer "F.Cu") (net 15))
 (segment (start 237.75 99.25) (end 238.5 98.5) (width 0.2) (layer "F.Cu") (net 15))
 (via (at 240.5 95) (size 0.6) (drill 0.3) (layers "F.Cu" "B.Cu") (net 15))
 (via (at 238.5 98.5) (size 0.6) (drill 0.3) (layers "F.Cu" "B.Cu") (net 15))
 (segment (start 238.5 98.5) (end 238.5 97) (width 0.2) (layer "B.Cu") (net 15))
 (segment (start 238.5 97) (end 240.5 95) (width 0.2) (layer "B.Cu") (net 15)))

